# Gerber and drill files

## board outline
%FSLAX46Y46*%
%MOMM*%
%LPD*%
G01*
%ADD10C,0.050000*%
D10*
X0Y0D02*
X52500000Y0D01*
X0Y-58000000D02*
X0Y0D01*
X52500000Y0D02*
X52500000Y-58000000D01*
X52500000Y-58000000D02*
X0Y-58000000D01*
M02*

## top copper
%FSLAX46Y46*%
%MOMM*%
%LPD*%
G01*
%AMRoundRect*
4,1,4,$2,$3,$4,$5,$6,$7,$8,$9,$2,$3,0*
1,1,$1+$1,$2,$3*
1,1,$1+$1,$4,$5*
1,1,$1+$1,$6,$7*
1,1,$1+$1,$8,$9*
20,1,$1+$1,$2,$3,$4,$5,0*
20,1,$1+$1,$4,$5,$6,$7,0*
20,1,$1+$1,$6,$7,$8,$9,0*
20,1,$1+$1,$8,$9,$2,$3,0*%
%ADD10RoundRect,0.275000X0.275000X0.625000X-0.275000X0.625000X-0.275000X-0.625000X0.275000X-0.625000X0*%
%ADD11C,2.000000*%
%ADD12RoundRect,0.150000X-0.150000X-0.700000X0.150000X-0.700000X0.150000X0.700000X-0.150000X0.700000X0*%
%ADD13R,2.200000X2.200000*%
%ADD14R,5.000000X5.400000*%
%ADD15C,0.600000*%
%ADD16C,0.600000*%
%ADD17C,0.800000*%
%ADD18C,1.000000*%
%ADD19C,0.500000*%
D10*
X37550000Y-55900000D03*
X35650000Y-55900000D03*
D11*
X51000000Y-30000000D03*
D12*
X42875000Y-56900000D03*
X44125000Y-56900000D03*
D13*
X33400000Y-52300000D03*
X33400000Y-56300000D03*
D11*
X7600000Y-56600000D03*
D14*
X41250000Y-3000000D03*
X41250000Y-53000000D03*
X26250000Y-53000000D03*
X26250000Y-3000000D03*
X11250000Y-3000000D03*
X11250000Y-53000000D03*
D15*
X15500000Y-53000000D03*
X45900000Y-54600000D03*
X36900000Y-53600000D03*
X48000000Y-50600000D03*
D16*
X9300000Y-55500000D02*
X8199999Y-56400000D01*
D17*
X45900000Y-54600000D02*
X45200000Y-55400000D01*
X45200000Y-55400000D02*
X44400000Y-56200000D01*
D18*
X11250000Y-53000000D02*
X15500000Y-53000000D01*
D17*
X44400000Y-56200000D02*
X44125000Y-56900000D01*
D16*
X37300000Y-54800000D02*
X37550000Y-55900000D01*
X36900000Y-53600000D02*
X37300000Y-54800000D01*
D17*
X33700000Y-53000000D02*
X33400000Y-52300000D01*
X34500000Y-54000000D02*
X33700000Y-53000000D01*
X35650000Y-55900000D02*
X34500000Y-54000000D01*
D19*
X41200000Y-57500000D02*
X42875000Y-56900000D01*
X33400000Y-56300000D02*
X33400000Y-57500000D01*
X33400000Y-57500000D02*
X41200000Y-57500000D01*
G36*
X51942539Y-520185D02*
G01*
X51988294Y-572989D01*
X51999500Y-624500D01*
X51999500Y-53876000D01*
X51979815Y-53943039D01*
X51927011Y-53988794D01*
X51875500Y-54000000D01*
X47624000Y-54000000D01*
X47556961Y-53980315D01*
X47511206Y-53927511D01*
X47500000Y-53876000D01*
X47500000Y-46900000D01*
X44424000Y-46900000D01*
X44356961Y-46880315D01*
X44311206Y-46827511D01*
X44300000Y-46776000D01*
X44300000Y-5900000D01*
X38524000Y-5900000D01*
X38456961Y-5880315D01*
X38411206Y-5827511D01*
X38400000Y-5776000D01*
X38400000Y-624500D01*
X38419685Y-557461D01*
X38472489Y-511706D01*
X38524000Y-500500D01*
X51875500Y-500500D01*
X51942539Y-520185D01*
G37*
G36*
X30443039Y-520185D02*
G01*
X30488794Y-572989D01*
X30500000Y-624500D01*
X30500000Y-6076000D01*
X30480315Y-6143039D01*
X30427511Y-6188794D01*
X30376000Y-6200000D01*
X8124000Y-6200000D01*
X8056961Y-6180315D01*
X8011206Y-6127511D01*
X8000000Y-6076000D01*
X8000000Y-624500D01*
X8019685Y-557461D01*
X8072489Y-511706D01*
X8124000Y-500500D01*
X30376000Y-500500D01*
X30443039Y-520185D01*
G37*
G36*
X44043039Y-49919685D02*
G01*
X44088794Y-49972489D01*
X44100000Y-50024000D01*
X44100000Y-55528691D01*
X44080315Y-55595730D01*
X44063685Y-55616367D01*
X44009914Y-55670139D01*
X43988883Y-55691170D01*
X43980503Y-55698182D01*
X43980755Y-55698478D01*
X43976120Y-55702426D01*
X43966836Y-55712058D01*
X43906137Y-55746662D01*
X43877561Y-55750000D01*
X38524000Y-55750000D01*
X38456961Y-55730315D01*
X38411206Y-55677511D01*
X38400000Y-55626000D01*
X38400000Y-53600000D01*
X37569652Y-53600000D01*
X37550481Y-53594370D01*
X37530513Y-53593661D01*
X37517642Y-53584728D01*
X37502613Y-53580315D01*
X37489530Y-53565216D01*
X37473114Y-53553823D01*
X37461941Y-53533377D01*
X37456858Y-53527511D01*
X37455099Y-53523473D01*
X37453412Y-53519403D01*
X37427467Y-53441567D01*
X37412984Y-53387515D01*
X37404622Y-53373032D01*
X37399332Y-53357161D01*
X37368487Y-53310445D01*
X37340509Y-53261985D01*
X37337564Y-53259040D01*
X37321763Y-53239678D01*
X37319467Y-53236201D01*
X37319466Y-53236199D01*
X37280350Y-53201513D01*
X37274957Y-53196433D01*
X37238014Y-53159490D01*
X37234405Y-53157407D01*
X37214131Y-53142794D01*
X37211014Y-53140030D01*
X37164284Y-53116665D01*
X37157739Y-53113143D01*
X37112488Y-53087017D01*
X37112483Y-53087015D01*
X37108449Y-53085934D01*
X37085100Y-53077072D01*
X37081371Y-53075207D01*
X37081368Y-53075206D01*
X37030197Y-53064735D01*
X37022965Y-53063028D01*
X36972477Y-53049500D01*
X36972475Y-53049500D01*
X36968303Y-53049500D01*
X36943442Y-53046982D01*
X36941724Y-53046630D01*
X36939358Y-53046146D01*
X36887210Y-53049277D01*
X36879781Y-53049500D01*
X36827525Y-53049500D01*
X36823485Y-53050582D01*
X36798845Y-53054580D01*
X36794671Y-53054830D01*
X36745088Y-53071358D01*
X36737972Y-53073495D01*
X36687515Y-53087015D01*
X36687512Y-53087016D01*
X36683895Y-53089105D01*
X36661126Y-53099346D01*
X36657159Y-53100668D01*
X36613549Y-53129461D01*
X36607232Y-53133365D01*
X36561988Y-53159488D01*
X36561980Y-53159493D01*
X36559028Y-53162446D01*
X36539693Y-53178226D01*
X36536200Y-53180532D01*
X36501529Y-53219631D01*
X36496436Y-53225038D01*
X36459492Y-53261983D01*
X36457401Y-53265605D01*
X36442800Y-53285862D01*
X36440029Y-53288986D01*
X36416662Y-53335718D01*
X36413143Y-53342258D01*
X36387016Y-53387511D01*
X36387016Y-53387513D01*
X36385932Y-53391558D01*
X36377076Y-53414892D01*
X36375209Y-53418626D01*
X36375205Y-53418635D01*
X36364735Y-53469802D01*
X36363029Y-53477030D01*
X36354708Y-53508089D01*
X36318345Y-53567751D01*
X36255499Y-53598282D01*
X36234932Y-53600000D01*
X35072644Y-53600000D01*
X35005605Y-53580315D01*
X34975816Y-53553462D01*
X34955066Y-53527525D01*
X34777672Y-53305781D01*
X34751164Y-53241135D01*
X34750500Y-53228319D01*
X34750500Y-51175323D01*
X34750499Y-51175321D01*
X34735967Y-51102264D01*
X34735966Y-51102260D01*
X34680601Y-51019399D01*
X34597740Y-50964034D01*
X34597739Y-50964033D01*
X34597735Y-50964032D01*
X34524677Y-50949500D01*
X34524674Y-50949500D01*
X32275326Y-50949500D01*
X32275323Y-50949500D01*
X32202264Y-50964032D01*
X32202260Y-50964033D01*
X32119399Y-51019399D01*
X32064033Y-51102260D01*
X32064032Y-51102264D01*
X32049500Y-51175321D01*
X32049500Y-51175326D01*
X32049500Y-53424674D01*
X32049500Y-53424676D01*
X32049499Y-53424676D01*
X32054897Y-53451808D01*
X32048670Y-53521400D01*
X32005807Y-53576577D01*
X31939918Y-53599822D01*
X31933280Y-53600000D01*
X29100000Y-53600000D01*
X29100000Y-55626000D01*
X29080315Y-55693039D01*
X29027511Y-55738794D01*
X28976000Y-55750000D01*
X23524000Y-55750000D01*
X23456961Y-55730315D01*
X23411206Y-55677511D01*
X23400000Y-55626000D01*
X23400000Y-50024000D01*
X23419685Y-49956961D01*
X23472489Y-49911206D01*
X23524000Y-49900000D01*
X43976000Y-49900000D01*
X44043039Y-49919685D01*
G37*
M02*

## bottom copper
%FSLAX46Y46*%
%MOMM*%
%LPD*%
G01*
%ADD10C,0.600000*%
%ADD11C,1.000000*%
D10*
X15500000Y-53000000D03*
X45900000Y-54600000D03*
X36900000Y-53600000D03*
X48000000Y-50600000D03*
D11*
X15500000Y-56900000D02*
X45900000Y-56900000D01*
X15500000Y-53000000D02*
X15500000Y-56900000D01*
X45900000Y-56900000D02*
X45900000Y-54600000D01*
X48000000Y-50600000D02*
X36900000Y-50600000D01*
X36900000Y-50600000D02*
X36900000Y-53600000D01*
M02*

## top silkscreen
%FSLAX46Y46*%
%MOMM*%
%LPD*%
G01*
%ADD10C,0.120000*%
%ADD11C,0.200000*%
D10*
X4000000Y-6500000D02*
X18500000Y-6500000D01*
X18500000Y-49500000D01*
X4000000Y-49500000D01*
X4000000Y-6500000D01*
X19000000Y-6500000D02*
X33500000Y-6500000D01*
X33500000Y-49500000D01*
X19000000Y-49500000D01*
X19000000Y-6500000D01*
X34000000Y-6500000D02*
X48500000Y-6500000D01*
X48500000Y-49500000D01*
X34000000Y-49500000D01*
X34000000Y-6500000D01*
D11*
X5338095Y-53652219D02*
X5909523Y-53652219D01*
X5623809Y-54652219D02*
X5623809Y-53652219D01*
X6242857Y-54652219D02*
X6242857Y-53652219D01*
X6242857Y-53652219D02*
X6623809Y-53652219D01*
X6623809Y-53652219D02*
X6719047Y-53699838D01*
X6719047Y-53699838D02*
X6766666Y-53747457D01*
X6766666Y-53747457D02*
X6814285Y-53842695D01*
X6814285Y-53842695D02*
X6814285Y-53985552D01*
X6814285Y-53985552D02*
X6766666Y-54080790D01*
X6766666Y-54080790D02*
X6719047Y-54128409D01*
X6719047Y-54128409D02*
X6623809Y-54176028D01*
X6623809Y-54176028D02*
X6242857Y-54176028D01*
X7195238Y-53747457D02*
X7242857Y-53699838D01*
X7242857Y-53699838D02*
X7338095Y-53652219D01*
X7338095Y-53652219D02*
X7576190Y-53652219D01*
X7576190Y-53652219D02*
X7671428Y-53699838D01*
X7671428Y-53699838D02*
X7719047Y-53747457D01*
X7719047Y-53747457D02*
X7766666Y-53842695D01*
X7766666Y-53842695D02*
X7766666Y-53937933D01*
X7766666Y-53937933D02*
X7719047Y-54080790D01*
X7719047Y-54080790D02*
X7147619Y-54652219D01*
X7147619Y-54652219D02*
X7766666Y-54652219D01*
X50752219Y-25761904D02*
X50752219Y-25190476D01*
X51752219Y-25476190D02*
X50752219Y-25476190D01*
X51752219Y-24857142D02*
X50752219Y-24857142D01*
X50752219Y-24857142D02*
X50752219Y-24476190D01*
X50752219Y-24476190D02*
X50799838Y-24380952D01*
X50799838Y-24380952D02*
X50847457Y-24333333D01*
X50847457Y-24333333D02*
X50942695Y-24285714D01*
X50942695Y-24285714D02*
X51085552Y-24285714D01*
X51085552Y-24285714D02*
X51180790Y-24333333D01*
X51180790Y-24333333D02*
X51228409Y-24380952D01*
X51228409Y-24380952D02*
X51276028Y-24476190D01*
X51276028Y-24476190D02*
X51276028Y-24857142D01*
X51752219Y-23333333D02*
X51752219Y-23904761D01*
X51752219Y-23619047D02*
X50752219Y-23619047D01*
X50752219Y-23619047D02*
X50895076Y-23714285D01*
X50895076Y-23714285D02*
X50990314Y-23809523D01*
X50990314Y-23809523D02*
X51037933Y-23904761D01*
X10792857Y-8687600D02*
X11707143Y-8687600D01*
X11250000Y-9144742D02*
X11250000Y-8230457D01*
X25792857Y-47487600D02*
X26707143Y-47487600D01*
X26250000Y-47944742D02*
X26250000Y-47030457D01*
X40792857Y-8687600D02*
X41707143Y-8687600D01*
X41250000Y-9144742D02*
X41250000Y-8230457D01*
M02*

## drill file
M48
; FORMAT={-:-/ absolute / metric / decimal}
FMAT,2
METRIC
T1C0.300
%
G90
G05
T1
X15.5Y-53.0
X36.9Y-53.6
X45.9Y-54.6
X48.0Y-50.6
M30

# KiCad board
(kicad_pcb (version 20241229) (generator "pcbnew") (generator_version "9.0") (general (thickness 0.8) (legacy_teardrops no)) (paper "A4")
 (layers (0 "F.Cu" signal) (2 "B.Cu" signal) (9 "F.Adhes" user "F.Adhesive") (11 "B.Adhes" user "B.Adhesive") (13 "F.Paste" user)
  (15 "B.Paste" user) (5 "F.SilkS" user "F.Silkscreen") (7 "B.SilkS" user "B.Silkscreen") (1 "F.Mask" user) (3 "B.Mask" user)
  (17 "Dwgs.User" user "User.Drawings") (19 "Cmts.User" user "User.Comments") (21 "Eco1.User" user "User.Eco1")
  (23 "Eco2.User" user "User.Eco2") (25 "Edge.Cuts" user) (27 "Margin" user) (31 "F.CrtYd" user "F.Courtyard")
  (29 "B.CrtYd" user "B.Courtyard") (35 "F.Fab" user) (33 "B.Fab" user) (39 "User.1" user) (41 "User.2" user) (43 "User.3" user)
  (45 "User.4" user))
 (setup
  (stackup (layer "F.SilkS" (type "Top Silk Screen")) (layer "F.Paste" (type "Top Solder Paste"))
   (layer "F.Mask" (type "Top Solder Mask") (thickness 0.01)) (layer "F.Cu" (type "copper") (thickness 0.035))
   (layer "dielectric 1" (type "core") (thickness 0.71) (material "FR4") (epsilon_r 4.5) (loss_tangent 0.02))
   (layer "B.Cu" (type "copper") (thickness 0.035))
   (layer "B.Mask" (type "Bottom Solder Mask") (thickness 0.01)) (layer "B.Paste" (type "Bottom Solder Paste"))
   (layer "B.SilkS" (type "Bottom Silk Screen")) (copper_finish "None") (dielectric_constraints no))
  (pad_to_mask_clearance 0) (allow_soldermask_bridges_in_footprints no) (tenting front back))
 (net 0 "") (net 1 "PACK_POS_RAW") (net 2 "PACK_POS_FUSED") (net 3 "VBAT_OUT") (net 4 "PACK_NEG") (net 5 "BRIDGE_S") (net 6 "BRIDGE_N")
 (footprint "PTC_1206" (layer "F.Cu") (at 36.6 55.9 180)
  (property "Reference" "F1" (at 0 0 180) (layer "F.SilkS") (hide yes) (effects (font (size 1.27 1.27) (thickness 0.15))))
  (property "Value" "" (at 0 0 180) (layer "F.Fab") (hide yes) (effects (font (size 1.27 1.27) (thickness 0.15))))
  (pad "1" smd roundrect (at -0.95 0 180) (size 1.1 1.8) (layers "F.Cu" "F.Mask" "F.Paste") (roundrect_rratio 0.25) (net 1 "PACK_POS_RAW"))
  (pad "2" smd roundrect (at 0.95 0 180) (size 1.1 1.8) (layers "F.Cu" "F.Mask" "F.Paste") (roundrect_rratio 0.25) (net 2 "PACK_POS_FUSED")))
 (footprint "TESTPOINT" (layer "F.Cu") (at 51 30)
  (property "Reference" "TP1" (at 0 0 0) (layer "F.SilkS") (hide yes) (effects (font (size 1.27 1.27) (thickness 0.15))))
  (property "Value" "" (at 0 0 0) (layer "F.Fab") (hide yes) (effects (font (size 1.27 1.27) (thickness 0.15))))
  (pad "1" smd circle (at 0 0) (size 2 2) (layers "F.Cu" "F.Mask") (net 1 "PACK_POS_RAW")))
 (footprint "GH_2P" (layer "F.Cu") (at 43.5 56.9)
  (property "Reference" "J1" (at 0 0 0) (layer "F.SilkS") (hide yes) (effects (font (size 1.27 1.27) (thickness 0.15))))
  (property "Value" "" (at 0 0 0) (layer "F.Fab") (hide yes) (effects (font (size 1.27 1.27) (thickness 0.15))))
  (pad "1" smd roundrect (at -0.625 0) (size 0.6 1.7) (layers "F.Cu" "F.Mask" "F.Paste") (roundrect_rratio 0.25) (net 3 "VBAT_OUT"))
  (pad "2" smd roundrect (at 0.625 0) (size 0.6 1.7) (layers "F.Cu" "F.Mask" "F.Paste") (roundrect_rratio 0.25) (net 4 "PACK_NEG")))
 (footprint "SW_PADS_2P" (layer "F.Cu") (at 33.4 54.3)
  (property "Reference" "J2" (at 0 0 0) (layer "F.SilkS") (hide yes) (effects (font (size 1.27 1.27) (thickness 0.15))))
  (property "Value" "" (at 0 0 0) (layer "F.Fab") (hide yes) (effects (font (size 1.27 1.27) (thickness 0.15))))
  (pad "1" smd rect (at 0 -2) (size 2.2 2.2) (layers "F.Cu" "F.Mask" "F.Paste") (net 2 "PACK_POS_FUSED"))
  (pad "2" smd rect (at 0 2) (size 2.2 2.2) (layers "F.Cu" "F.Mask" "F.Paste") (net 3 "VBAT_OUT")))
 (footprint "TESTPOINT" (layer "F.Cu") (at 7.6 56.6)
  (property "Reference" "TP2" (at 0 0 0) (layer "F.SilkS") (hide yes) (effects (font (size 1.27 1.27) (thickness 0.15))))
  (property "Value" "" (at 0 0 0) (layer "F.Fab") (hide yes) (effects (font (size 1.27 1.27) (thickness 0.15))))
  (pad "1" smd circle (at 0 0) (size 2 2) (layers "F.Cu" "F.Mask") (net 4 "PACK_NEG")))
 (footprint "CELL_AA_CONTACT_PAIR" (layer "F.Cu") (at 41.25 28)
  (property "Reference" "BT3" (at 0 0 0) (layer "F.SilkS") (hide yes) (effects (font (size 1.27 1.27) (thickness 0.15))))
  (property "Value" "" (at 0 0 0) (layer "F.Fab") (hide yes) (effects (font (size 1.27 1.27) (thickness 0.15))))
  (pad "1" smd rect (at 0 -25) (size 5 5.4) (layers "F.Cu" "F.Mask" "F.Paste") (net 1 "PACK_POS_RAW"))
  (pad "2" smd rect (at 0 25) (size 5 5.4) (layers "F.Cu" "F.Mask" "F.Paste") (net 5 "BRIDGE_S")))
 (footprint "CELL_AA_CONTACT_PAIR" (layer "F.Cu") (at 26.25 28 180)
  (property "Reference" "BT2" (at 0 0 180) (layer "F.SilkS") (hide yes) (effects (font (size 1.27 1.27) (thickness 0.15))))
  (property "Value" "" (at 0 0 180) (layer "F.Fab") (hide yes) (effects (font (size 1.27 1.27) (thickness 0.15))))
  (pad "1" smd rect (at 0 -25 180) (size 5 5.4) (layers "F.Cu" "F.Mask" "F.Paste") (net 5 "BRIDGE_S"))
  (pad "2" smd rect (at 0 25 180) (size 5 5.4) (layers "F.Cu" "F.Mask" "F.Paste") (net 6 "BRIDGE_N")))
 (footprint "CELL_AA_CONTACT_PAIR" (layer "F.Cu") (at 11.25 28)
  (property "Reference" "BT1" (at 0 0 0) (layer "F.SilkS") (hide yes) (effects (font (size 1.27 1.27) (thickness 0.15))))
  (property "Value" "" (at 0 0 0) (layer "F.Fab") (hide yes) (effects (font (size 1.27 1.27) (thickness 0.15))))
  (pad "1" smd rect (at 0 -25) (size 5 5.4) (layers "F.Cu" "F.Mask" "F.Paste") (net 6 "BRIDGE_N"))
  (pad "2" smd rect (at 0 25) (size 5 5.4) (layers "F.Cu" "F.Mask" "F.Paste") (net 4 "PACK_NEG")))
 (gr_rect (start 4 6.5) (end 18.5 49.5) (stroke (width 0.12) (type default)) (fill no) (layer "F.SilkS"))
 (gr_rect (start 19 6.5) (end 33.5 49.5) (stroke (width 0.12) (type default)) (fill no) (layer "F.SilkS"))
 (gr_rect (start 34 6.5) (end 48.5 49.5) (stroke (width 0.12) (type default)) (fill no) (layer "F.SilkS"))
 (gr_line (start 0 0) (end 52.5 0) (stroke (width 0.05) (type default)) (layer "Edge.Cuts"))
 (gr_line (start 0 58) (end 0 0) (stroke (width 0.05) (type default)) (layer "Edge.Cuts"))
 (gr_line (start 52.5 0) (end 52.5 58) (stroke (width 0.05) (type default)) (layer "Edge.Cuts"))
 (gr_line (start 52.5 58) (end 0 58) (stroke (width 0.05) (type default)) (layer "Edge.Cuts"))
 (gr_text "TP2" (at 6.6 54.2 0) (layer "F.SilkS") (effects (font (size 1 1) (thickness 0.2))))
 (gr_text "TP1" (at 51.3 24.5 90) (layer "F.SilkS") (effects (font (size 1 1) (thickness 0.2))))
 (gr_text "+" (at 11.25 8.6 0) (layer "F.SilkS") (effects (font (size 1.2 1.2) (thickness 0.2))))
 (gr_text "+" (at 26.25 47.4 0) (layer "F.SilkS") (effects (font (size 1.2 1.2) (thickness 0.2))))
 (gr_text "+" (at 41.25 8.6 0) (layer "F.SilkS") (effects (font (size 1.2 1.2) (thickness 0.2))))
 (segment (start 9.3 55.5) (end 8.199999 56.4) (width 0.6) (layer "F.Cu") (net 4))
 (segment (start 45.9 54.6) (end 45.2 55.4) (width 0.8) (layer "F.Cu") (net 4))
 (segment (start 45.2 55.4) (end 44.4 56.2) (width 0.8) (layer "F.Cu") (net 4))
 (segment (start 11.25 53) (end 15.5 53) (width 1) (layer "F.Cu") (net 4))
 (segment (start 44.4 56.2) (end 44.125 56.9) (width 0.8) (layer "F.Cu") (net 4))
 (via (at 15.5 53) (size 0.6) (drill 0.3) (layers "F.Cu" "B.Cu") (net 4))
 (via (at 45.9 54.6) (size 0.6) (drill 0.3) (layers "F.Cu" "B.Cu") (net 4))
 (segment (start 15.5 56.9) (end 45.9 56.9) (width 1) (layer "B.Cu") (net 4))
 (segment (start 15.5 53) (end 15.5 56.9) (width 1) (layer "B.Cu") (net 4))
 (segment (start 45.9 56.9) (end 45.9 54.6) (width 1) (layer "B.Cu") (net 4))
 (segment (start 37.3 54.8) (end 37.55 55.9) (width 0.6) (layer "F.Cu") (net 1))
 (segment (start 36.9 53.6) (end 37.3 54.8) (width 0.6) (layer "F.Cu") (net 1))
 (via (at 36.9 53.6) (size 0.6) (drill 0.3) (layers "F.Cu" "B.Cu") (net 1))
 (via (at 48 50.6) (size 0.6) (drill 0.3) (layers "F.Cu" "B.Cu") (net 1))
 (segment (start 48 50.6) (end 36.9 50.6) (width 1) (layer "B.Cu") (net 1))
 (segment (start 36.9 50.6) (end 36.9 53.6) (width 1) (layer "B.Cu") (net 1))
 (segment (start 33.7 53) (end 33.4 52.3) (width 0.8) (layer "F.Cu") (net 2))
 (segment (start 34.5 54) (end 33.7 53) (width 0.8) (layer "F.Cu") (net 2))
 (segment (start 35.65 55.9) (end 34.5 54) (width 0.8) (layer "F.Cu") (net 2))
 (segment (start 41.2 57.5) (end 42.875 56.9) (width 0.5) (layer "F.Cu") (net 3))
 (segment (start 33.4 56.3) (end 33.4 57.5) (width 0.5) (layer "F.Cu") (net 3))
 (segment (start 33.4 57.5) (end 41.2 57.5) (width 0.5) (layer "F.Cu") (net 3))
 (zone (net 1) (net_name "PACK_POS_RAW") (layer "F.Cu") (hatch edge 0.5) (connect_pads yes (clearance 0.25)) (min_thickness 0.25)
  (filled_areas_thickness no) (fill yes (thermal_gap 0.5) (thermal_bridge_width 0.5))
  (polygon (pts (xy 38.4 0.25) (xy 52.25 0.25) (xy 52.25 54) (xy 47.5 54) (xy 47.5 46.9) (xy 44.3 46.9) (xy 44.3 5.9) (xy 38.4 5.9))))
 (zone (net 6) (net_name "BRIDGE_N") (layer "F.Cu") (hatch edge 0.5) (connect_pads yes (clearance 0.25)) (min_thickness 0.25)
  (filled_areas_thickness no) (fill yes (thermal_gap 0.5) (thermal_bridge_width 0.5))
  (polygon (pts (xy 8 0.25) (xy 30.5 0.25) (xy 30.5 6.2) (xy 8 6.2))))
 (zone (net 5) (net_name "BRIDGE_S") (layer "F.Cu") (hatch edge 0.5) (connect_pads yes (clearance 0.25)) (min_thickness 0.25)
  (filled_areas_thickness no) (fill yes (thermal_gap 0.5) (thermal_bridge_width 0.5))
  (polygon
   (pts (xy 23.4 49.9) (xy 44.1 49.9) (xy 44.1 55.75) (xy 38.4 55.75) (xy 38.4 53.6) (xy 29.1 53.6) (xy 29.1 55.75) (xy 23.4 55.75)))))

